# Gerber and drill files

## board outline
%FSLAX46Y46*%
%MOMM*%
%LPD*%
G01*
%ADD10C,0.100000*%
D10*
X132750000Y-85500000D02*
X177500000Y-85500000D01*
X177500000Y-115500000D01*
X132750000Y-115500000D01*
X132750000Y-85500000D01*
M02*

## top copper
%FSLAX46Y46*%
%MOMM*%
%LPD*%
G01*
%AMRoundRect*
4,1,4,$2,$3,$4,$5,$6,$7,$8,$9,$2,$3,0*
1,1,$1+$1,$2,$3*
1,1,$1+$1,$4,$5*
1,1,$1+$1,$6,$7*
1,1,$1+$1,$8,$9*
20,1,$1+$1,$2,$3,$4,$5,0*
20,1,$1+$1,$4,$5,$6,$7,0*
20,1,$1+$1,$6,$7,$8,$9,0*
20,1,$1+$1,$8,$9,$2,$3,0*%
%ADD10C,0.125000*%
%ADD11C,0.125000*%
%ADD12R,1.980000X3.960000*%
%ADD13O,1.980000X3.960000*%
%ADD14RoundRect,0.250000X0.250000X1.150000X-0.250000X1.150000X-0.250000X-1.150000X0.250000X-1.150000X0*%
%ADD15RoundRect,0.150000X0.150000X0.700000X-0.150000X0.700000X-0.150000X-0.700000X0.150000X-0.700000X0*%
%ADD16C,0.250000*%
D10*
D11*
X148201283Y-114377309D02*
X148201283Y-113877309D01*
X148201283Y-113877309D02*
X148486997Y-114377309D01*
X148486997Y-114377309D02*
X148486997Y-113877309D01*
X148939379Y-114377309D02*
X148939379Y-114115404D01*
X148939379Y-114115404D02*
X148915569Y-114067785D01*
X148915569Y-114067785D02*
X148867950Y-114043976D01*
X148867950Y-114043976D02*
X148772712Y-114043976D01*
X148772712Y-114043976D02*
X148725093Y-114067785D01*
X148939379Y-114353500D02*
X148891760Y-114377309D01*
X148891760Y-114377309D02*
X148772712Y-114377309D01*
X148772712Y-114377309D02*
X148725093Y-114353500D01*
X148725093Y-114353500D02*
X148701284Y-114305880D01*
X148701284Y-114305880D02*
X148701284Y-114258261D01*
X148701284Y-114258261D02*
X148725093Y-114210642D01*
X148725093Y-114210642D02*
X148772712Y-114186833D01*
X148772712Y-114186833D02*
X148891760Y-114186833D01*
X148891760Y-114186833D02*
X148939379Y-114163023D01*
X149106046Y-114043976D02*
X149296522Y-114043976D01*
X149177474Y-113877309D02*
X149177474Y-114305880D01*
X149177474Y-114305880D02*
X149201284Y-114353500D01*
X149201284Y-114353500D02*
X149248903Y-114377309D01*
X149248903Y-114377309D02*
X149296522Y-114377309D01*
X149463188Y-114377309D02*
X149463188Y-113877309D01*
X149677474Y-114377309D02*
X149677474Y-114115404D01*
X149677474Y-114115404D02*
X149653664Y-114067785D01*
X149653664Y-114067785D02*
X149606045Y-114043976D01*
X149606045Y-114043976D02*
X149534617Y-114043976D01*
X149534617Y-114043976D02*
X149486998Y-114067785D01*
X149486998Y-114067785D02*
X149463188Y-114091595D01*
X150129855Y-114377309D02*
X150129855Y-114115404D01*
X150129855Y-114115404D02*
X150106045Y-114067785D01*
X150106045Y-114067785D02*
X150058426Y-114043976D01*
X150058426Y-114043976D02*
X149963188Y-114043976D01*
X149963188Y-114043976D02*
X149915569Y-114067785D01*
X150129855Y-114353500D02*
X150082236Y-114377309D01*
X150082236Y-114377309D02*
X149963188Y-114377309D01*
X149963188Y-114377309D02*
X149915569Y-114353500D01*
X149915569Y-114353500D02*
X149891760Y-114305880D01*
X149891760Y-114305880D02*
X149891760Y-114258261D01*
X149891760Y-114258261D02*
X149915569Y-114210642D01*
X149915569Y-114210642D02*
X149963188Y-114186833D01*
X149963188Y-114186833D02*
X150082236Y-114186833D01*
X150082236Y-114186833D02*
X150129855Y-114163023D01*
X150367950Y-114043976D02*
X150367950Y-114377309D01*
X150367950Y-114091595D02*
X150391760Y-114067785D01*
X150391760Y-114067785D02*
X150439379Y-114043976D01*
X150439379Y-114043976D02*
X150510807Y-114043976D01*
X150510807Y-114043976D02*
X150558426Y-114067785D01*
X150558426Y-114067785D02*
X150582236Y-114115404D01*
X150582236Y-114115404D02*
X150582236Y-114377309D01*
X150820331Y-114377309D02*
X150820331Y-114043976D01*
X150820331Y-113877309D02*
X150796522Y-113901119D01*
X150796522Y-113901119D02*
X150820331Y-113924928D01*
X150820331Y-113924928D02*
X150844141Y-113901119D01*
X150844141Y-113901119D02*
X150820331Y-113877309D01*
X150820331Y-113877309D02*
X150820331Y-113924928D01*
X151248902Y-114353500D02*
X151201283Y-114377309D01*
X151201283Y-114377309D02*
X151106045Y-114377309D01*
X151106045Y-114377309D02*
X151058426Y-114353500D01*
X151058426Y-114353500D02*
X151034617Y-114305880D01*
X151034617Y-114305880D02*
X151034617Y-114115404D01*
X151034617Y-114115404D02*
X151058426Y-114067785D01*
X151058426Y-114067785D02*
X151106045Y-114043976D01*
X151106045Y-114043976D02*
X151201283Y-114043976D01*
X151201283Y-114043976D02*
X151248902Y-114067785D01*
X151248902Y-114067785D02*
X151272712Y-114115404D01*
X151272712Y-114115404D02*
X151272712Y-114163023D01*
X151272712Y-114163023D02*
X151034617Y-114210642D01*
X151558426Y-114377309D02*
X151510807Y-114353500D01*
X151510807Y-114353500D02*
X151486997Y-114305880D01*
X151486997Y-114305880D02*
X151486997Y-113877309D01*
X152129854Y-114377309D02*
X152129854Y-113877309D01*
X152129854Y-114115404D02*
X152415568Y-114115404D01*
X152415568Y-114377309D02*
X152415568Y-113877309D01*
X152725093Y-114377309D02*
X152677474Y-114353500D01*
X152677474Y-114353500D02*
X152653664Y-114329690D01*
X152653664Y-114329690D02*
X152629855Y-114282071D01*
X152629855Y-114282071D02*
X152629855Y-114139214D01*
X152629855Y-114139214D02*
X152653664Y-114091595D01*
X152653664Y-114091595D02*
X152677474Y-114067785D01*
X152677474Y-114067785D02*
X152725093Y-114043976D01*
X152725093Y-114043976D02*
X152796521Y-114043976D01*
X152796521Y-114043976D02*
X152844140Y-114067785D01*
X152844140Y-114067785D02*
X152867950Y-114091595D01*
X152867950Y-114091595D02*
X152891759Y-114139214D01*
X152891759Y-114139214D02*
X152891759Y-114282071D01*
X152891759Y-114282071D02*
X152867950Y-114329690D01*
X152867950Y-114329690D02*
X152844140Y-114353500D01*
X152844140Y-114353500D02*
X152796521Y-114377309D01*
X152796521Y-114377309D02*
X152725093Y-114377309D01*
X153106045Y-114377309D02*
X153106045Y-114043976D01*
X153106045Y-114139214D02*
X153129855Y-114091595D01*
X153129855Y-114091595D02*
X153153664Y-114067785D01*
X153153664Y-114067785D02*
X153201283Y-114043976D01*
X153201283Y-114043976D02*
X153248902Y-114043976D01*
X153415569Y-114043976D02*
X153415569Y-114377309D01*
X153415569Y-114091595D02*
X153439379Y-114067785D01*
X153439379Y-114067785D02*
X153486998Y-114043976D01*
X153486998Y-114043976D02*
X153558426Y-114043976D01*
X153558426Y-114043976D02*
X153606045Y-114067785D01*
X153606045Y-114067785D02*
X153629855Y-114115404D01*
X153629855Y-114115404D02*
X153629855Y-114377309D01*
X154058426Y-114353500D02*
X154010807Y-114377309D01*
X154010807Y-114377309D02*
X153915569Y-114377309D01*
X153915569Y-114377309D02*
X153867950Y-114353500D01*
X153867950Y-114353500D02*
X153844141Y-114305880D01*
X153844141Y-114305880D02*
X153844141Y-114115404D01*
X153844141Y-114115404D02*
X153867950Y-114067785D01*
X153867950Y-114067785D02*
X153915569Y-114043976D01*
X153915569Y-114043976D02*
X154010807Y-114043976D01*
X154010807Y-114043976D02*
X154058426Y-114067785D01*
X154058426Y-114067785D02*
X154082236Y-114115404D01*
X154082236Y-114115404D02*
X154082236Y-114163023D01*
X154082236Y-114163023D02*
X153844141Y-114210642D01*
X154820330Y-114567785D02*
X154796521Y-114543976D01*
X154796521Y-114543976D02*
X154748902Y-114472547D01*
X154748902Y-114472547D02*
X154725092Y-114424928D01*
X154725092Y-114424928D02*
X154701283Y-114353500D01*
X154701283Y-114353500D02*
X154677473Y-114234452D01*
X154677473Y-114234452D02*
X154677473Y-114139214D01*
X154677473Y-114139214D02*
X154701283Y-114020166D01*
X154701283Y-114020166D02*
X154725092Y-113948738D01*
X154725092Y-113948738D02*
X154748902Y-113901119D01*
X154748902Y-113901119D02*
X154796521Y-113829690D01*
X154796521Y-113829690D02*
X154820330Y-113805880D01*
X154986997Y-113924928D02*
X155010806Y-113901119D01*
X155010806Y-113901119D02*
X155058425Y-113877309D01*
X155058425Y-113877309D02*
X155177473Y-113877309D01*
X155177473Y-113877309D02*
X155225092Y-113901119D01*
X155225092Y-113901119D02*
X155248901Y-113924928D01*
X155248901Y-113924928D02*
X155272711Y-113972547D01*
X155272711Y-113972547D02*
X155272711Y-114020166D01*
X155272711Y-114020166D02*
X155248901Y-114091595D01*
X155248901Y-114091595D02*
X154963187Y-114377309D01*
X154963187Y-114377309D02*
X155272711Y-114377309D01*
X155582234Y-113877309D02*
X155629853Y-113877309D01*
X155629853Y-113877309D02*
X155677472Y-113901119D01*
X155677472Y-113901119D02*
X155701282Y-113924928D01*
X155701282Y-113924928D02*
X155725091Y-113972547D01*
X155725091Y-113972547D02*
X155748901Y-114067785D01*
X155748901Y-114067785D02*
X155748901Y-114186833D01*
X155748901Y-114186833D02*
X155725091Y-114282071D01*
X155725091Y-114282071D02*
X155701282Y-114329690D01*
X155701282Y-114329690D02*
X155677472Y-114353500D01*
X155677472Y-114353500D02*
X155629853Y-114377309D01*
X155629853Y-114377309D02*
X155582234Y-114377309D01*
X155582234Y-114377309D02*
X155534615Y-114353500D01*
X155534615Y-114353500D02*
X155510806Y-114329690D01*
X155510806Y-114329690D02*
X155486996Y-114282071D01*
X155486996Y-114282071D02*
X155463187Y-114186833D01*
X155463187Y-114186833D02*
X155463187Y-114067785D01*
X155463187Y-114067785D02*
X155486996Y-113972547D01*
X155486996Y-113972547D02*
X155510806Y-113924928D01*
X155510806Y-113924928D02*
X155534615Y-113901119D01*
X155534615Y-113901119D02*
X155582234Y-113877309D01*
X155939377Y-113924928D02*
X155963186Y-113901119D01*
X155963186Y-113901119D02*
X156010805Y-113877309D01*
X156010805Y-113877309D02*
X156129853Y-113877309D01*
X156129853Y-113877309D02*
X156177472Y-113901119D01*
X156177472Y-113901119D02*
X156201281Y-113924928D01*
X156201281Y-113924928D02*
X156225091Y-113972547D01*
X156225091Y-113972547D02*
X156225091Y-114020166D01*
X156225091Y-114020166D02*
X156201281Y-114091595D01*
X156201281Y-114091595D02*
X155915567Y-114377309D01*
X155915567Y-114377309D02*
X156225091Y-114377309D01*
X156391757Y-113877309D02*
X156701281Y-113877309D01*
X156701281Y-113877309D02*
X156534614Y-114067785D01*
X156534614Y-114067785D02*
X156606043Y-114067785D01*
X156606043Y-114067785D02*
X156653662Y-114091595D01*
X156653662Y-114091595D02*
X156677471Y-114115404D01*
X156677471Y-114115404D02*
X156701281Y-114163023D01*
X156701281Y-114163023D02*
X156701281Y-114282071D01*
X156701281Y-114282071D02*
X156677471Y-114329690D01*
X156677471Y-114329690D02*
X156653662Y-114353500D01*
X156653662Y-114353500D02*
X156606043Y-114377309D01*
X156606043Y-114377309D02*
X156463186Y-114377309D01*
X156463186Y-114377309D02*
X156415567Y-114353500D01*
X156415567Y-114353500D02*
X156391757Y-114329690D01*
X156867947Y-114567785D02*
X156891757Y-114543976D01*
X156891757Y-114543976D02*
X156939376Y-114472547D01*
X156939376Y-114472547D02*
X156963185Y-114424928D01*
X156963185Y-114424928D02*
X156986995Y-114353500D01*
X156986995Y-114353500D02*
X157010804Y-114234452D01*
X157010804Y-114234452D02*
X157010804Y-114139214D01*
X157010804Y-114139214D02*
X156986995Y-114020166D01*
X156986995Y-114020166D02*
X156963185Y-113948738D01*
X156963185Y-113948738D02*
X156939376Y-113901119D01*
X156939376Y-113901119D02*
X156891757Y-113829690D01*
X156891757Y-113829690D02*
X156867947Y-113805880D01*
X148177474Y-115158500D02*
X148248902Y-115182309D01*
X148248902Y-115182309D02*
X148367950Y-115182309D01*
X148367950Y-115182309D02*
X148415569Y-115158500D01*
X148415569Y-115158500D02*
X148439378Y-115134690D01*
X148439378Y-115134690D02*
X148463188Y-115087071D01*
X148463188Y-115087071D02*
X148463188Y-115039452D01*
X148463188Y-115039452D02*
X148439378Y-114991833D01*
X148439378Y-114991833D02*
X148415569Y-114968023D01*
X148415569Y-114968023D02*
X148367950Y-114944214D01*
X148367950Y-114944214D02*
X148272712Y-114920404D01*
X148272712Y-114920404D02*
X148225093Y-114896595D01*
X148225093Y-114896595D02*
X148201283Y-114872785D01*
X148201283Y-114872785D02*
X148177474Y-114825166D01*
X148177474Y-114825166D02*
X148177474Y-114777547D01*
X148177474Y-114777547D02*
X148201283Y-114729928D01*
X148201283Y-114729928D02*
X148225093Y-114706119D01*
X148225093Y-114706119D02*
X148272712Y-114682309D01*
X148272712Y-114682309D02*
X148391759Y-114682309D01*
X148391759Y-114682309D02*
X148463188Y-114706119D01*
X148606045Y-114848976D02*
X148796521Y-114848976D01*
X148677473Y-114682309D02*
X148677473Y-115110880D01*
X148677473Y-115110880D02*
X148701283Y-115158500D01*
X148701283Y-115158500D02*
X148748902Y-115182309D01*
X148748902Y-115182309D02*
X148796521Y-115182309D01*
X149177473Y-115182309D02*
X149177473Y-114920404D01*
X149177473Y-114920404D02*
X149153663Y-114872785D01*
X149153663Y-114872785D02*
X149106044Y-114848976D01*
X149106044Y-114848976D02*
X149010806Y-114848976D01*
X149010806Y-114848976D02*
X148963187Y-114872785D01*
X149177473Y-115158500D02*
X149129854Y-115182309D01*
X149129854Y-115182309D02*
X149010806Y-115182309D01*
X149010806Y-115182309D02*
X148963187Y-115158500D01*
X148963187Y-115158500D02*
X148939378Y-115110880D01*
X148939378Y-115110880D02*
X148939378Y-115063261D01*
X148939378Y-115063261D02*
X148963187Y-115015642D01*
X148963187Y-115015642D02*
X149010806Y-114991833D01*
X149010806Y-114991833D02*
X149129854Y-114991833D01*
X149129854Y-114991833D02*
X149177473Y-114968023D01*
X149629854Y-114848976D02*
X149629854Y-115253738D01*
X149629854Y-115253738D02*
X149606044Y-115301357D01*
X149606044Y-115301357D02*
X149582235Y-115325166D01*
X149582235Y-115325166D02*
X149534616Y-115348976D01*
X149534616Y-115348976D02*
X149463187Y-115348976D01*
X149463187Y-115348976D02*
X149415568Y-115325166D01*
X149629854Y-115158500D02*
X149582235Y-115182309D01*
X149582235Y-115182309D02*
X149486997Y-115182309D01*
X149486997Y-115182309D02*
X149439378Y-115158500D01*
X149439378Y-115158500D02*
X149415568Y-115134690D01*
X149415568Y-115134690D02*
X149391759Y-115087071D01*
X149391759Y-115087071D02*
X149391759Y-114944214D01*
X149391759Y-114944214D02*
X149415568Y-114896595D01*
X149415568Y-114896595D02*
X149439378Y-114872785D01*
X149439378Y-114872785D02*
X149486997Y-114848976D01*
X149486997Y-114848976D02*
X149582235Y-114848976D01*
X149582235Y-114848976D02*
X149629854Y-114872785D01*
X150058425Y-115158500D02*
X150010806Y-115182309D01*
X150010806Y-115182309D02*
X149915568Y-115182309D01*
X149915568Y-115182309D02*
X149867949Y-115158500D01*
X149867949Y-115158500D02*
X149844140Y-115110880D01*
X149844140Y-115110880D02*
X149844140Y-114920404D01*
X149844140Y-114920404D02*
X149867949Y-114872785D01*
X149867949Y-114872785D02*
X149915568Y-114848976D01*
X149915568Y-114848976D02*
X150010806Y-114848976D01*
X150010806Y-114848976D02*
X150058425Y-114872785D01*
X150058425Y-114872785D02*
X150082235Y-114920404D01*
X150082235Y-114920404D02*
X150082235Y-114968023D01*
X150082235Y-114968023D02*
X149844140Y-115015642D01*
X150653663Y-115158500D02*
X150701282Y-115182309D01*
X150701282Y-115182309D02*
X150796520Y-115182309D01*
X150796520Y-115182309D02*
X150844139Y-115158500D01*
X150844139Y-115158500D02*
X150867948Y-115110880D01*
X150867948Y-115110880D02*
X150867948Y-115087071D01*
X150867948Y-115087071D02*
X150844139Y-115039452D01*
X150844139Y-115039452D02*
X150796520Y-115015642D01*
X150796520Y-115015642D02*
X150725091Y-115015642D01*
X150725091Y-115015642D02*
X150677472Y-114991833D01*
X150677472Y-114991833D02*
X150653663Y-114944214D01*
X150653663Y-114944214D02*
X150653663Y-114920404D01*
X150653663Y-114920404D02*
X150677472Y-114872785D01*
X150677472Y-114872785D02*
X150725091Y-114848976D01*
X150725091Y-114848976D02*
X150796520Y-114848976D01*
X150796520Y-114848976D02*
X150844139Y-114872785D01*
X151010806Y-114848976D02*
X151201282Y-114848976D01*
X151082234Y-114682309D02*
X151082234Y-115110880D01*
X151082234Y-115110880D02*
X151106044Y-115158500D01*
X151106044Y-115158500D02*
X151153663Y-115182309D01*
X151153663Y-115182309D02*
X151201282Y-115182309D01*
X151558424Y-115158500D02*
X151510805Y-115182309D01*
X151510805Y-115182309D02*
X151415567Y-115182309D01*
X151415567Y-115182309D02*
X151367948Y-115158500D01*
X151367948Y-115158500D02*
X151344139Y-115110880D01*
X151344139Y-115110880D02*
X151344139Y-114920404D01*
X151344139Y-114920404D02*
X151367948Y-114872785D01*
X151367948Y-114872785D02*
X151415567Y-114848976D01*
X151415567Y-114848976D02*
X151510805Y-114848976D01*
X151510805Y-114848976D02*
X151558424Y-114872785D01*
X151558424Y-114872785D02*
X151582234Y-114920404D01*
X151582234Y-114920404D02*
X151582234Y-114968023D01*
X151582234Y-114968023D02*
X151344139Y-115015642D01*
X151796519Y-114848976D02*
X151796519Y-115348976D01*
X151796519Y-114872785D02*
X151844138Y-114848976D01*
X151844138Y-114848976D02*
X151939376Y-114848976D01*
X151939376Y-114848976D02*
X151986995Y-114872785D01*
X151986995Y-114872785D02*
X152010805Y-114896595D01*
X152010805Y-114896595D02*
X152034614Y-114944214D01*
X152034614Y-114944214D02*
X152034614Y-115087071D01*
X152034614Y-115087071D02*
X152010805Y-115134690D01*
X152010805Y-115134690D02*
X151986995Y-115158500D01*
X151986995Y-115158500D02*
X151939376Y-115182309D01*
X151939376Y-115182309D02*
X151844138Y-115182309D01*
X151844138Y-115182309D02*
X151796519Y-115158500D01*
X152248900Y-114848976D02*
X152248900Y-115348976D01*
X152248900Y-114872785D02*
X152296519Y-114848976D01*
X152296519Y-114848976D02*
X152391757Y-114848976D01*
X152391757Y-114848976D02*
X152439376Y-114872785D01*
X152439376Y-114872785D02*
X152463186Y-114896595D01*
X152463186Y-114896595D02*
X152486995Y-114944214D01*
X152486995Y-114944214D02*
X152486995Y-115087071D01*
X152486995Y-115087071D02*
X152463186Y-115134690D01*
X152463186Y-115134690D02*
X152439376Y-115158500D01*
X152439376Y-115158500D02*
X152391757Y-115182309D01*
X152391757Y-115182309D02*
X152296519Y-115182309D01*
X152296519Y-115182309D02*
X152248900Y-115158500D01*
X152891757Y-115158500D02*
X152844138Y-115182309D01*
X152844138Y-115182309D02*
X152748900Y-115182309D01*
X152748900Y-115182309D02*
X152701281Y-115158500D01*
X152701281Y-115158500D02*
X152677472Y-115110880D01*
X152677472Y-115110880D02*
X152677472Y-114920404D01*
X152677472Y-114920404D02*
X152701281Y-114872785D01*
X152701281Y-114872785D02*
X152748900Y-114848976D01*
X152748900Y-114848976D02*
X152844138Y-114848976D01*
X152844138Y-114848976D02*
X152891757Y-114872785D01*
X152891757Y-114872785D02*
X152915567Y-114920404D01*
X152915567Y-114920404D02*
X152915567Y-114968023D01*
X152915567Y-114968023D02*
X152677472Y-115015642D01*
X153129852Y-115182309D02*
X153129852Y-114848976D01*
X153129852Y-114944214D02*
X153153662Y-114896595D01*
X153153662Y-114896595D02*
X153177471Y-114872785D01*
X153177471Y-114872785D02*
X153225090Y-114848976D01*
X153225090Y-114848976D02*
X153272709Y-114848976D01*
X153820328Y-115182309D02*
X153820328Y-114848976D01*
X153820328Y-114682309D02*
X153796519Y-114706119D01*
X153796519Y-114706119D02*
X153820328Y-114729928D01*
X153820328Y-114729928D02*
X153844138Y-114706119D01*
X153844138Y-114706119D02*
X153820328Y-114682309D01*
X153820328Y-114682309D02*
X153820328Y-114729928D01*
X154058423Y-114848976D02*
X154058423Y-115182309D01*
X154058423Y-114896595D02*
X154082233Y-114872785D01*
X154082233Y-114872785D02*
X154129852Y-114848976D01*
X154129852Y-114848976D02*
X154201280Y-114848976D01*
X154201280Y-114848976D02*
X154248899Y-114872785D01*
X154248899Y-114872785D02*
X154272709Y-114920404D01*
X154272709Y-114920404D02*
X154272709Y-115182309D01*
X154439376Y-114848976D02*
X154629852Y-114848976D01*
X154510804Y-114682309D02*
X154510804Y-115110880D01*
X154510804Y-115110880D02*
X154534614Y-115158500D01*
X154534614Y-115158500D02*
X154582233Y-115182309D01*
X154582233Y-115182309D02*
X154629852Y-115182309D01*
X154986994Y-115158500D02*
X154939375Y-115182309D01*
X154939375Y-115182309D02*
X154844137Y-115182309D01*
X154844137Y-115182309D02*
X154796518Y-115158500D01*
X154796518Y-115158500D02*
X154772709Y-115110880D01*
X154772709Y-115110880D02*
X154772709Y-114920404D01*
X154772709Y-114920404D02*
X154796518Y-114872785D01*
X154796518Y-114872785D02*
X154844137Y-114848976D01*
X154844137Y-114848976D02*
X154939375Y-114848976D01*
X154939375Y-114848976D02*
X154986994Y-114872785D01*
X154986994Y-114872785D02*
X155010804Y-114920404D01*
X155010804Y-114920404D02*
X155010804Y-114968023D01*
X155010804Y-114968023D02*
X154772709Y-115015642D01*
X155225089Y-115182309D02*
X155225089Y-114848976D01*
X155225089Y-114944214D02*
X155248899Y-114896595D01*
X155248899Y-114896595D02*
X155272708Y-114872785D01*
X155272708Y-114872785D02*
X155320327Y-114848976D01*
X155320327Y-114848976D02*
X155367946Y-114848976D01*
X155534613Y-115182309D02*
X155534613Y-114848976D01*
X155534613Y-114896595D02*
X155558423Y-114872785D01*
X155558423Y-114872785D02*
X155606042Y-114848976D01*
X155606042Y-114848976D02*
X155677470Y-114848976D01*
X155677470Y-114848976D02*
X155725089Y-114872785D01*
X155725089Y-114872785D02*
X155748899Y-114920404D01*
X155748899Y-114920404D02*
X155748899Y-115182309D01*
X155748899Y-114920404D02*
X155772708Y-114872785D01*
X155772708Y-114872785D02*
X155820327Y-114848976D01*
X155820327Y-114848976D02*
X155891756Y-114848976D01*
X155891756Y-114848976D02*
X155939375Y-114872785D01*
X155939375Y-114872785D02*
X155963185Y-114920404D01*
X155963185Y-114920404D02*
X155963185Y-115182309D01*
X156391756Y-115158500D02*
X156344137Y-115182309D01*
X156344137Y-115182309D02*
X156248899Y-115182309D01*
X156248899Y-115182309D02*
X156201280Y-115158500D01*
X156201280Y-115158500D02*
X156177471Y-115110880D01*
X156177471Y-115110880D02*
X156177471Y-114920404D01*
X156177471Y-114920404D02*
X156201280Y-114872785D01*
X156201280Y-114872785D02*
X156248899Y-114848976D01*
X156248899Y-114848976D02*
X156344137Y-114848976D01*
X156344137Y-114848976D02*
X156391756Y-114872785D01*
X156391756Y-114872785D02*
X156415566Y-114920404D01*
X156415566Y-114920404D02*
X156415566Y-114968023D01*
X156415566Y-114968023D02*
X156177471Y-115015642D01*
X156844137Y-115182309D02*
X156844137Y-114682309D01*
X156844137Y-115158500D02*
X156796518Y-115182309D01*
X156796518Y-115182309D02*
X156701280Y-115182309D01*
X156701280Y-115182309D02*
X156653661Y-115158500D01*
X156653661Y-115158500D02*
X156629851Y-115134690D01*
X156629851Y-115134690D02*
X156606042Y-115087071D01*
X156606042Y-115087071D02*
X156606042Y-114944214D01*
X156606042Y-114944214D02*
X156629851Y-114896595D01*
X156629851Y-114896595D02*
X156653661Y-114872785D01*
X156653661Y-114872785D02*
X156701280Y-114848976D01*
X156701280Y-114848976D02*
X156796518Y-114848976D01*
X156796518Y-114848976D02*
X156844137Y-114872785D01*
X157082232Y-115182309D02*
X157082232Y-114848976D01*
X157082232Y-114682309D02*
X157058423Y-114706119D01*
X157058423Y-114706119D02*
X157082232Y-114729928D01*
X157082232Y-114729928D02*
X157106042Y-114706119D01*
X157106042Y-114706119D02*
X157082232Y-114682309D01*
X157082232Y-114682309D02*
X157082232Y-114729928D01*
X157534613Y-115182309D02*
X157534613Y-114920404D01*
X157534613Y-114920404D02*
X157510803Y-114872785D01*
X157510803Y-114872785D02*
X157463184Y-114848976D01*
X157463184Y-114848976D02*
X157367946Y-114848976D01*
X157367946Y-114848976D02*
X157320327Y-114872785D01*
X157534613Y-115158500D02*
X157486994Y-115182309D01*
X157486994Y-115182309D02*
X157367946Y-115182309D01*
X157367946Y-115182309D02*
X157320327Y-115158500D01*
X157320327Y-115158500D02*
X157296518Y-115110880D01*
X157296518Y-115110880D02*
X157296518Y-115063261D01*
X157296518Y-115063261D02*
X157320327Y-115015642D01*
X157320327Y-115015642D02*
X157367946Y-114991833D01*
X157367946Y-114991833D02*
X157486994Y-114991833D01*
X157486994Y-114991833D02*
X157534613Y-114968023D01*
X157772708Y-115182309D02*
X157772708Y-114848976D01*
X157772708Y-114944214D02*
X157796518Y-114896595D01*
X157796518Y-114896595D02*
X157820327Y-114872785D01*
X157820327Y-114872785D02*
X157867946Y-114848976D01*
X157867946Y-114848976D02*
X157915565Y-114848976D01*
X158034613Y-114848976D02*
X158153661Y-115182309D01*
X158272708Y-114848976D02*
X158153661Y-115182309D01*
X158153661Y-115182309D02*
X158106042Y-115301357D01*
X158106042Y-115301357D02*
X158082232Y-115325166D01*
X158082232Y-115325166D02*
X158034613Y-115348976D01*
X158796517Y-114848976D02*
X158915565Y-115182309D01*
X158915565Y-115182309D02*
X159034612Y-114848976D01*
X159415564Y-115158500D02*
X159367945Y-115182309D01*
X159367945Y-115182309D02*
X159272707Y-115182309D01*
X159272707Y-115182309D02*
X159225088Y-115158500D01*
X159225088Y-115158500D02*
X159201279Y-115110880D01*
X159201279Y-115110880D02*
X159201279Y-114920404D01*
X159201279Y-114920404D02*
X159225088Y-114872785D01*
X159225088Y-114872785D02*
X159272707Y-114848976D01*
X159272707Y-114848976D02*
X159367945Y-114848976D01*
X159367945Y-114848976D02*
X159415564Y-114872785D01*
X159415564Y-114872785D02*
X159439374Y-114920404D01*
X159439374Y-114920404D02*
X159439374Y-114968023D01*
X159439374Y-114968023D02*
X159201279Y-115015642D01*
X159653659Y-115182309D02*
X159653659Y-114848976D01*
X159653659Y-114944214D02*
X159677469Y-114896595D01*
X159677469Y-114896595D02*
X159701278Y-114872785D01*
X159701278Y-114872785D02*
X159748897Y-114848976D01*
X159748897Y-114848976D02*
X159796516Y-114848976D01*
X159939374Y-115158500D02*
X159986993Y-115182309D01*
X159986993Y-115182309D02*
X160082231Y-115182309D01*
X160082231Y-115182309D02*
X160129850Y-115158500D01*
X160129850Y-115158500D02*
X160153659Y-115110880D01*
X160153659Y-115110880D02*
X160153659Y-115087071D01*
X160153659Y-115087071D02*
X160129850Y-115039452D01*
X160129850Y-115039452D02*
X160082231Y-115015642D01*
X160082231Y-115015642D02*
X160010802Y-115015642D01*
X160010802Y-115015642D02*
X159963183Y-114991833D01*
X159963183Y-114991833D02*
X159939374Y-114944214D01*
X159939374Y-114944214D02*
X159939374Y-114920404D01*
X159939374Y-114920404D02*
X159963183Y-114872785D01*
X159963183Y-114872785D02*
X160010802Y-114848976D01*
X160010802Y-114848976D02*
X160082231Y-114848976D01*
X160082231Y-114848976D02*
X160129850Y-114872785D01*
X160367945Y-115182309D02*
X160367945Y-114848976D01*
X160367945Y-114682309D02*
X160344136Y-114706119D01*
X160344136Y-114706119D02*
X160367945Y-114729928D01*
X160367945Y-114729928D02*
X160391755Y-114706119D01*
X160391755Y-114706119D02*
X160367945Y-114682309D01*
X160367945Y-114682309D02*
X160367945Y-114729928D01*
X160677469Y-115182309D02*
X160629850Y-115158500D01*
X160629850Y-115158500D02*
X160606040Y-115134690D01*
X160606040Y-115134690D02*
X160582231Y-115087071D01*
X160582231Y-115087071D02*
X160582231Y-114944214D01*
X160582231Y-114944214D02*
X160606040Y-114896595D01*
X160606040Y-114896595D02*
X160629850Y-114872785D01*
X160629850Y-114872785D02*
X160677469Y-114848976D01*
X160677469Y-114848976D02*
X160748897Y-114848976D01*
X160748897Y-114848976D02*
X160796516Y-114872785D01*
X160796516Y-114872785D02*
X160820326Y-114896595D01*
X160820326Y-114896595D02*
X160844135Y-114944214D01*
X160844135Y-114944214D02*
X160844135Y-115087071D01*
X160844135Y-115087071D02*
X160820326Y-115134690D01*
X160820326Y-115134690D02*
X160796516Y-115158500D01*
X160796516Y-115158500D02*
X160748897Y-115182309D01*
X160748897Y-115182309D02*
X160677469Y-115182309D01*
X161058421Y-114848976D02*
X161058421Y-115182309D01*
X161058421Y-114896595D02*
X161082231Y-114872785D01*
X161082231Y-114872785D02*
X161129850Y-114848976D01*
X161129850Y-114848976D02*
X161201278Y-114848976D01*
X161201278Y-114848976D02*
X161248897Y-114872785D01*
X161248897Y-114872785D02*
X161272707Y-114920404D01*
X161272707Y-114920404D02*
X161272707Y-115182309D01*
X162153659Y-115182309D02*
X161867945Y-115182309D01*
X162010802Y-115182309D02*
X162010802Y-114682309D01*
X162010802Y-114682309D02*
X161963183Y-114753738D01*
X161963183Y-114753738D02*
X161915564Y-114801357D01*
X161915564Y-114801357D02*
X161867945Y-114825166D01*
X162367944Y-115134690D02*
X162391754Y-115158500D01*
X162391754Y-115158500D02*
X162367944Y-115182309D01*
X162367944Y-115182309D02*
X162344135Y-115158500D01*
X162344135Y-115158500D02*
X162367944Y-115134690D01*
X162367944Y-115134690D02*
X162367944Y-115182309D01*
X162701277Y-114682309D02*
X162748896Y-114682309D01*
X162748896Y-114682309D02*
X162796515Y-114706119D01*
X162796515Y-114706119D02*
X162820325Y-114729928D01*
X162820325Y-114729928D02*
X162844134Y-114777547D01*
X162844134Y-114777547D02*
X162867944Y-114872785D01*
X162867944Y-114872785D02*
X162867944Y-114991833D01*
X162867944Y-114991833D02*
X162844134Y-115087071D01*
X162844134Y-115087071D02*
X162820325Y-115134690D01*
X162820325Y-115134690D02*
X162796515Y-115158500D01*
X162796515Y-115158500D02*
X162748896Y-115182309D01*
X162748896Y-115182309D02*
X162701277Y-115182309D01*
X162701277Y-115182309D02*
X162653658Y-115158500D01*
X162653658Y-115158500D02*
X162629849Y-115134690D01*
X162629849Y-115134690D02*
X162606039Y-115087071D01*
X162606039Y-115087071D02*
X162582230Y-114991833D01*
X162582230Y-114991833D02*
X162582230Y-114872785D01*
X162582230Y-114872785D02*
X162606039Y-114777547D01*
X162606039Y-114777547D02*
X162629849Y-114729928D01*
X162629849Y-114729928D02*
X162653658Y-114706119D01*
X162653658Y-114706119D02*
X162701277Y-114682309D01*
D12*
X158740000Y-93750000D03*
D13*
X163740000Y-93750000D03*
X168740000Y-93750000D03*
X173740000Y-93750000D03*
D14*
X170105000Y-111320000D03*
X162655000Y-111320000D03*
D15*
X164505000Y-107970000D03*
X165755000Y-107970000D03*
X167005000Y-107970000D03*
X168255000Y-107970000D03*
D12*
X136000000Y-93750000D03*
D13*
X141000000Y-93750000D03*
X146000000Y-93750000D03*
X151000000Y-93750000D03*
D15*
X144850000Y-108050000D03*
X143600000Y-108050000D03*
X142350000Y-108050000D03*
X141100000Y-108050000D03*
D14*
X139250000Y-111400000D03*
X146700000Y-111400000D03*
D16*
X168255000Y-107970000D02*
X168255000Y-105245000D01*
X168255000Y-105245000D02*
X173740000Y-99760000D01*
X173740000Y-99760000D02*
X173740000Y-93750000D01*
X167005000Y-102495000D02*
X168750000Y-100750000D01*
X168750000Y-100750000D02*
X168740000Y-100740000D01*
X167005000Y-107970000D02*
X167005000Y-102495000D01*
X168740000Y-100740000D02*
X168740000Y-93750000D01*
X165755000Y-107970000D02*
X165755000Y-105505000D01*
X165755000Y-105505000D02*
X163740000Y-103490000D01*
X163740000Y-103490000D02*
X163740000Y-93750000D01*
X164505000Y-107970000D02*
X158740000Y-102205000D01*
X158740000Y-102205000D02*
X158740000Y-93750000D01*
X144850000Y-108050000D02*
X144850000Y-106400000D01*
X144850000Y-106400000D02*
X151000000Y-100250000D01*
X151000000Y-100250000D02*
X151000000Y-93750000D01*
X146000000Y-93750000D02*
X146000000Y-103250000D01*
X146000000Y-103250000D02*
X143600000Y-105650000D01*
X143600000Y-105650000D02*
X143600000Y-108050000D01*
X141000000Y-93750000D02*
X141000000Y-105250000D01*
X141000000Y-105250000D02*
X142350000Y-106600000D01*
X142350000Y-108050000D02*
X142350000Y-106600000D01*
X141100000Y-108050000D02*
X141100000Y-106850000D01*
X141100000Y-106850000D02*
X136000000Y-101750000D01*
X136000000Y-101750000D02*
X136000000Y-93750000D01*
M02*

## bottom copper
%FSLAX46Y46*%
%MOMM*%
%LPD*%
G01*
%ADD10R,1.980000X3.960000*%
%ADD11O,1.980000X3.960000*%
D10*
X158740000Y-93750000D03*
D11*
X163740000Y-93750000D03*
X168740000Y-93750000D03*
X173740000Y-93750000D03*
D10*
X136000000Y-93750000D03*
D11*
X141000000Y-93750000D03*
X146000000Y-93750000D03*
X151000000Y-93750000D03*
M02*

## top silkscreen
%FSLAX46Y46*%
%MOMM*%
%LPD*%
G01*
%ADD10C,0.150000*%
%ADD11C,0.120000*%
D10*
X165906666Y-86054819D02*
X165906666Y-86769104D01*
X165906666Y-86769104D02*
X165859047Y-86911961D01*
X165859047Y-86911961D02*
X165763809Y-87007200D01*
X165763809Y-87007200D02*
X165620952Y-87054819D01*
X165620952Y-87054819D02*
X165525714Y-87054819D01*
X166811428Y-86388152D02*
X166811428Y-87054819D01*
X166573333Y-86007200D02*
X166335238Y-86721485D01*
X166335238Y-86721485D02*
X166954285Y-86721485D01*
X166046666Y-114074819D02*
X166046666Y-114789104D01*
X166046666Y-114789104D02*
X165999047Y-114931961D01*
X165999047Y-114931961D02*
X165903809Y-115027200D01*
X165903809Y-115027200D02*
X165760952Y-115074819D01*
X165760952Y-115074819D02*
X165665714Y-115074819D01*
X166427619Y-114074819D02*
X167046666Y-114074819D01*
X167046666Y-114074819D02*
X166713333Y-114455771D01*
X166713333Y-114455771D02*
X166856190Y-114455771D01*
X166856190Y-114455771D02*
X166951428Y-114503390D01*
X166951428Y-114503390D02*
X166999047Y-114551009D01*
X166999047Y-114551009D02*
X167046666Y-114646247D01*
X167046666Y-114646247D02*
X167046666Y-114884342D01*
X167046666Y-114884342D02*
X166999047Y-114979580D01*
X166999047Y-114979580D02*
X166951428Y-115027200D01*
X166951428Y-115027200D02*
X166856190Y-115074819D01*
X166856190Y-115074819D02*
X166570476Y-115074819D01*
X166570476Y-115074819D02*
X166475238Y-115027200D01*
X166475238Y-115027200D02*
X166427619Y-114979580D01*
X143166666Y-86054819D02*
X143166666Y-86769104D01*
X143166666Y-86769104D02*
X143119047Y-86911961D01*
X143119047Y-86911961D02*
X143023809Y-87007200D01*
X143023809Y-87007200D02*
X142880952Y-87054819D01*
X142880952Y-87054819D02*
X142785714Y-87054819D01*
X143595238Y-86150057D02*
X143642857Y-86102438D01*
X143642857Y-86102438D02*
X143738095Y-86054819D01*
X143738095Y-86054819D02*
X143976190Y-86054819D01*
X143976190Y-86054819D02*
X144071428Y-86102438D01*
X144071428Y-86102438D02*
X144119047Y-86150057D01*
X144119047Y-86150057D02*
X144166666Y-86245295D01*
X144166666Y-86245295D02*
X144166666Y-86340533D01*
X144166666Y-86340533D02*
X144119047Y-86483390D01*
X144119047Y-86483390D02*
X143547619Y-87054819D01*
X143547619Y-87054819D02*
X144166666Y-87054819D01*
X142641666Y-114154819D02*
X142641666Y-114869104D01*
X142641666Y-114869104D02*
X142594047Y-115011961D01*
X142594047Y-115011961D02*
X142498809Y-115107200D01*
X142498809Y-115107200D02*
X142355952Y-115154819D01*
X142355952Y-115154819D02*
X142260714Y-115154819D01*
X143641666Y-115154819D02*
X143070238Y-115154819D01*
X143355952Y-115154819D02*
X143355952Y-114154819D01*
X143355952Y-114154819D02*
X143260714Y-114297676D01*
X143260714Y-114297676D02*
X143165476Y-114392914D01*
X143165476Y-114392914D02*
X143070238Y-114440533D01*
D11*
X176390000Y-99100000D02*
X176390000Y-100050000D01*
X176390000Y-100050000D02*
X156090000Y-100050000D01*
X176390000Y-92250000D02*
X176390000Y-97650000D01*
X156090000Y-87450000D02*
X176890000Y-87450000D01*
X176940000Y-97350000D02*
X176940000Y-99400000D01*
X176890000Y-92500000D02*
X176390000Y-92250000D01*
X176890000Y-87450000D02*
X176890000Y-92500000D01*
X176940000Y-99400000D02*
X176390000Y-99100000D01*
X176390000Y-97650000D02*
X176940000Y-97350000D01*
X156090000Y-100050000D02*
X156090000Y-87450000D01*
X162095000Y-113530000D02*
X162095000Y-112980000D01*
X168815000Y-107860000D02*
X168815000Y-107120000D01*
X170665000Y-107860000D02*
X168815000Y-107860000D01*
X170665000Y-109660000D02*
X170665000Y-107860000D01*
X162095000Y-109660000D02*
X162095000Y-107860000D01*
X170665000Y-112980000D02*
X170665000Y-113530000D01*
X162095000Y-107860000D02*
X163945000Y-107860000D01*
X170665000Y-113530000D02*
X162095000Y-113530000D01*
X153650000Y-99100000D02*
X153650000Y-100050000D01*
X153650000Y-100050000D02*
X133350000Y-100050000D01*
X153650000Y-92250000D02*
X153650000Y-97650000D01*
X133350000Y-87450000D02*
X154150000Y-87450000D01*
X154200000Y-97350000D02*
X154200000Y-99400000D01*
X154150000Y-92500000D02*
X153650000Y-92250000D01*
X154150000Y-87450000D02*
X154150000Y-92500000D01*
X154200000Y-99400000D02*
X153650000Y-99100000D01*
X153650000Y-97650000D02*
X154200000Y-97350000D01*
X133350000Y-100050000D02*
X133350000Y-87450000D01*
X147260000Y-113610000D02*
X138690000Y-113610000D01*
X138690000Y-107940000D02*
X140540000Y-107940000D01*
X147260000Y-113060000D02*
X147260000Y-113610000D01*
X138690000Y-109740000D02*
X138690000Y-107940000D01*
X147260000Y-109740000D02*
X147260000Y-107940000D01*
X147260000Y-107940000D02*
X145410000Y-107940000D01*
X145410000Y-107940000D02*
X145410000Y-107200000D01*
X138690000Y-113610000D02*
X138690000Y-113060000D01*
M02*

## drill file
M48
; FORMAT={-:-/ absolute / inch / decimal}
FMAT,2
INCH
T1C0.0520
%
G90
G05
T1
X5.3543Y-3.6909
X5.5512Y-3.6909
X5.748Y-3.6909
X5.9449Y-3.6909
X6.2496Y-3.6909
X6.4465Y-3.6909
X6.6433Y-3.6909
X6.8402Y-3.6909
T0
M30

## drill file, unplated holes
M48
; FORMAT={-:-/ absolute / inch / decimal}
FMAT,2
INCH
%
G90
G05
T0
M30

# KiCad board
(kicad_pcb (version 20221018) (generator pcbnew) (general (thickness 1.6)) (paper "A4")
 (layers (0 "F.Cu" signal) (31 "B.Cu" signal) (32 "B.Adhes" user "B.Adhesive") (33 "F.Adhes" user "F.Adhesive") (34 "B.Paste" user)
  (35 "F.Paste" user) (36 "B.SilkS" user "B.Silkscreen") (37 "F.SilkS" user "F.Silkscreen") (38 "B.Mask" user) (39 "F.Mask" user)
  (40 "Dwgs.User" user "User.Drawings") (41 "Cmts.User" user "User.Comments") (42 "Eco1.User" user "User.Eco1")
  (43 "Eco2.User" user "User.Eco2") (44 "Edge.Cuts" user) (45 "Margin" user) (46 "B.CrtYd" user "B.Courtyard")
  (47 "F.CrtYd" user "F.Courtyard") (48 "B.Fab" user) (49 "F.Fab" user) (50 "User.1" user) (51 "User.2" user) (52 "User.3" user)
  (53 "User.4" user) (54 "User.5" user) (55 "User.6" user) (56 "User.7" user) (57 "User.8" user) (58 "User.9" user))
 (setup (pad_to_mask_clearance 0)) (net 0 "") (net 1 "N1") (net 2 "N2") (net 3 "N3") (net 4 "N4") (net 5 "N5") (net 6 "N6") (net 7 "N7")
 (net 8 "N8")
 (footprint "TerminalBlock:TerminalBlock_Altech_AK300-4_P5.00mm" (layer "F.Cu") (at 136 93.75)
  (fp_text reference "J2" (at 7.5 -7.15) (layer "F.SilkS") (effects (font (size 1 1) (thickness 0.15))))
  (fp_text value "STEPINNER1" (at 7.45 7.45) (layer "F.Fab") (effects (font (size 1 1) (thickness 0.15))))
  (fp_line (start -2.65 -6.3) (end 18.15 -6.3) (stroke (width 0.12) (type solid)) (layer "F.SilkS"))
  (fp_line (start -2.65 6.3) (end -2.65 -6.3) (stroke (width 0.12) (type solid)) (layer "F.SilkS"))
  (fp_line (start 17.65 -1.5) (end 17.65 3.9) (stroke (width 0.12) (type solid)) (layer "F.SilkS"))
  (fp_line (start 17.65 3.9) (end 18.2 3.6) (stroke (width 0.12) (type solid)) (layer "F.SilkS"))
  (fp_line (start 17.65 5.35) (end 17.65 6.3) (stroke (width 0.12) (type solid)) (layer "F.SilkS"))
  (fp_line (start 17.65 6.3) (end -2.65 6.3) (stroke (width 0.12) (type solid)) (layer "F.SilkS"))
  (fp_line (start 18.15 -6.3) (end 18.15 -1.25) (stroke (width 0.12) (type solid)) (layer "F.SilkS"))
  (fp_line (start 18.15 -1.25) (end 17.65 -1.5) (stroke (width 0.12) (type solid)) (layer "F.SilkS"))
  (fp_line (start 18.2 3.6) (end 18.2 5.65) (stroke (width 0.12) (type solid)) (layer "F.SilkS"))
  (fp_line (start 18.2 5.65) (end 17.65 5.35) (stroke (width 0.12) (type solid)) (layer "F.SilkS"))
  (pad "1" thru_hole rect (at 0 0) (size 1.98 3.96) (drill 1.32) (layers "*.Cu" "*.Mask") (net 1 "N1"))
  (pad "2" thru_hole oval (at 5 0) (size 1.98 3.96) (drill 1.32) (layers "*.Cu" "*.Mask") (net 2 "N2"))
  (pad "3" thru_hole oval (at 10 0) (size 1.98 3.96) (drill 1.32) (layers "*.Cu" "*.Mask") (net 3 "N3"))
  (pad "4" thru_hole oval (at 15 0) (size 1.98 3.96) (drill 1.32) (layers "*.Cu" "*.Mask") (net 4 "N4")))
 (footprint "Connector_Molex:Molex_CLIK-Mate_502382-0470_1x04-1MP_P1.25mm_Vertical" (layer "F.Cu") (at 142.975 110 180)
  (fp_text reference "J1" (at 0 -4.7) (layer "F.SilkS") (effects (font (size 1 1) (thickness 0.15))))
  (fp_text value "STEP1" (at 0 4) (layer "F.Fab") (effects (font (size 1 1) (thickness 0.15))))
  (fp_line (start -4.285 -3.61) (end 4.285 -3.61) (stroke (width 0.12) (type solid)) (layer "F.SilkS"))
  (fp_line (start -4.285 -3.06) (end -4.285 -3.61) (stroke (width 0.12) (type solid)) (layer "F.SilkS"))
  (fp_line (start -4.285 0.26) (end -4.285 2.06) (stroke (width 0.12) (type solid)) (layer "F.SilkS"))
  (fp_line (start -4.285 2.06) (end -2.435 2.06) (stroke (width 0.12) (type solid)) (layer "F.SilkS"))
  (fp_line (start -2.435 2.06) (end -2.435 2.8) (stroke (width 0.12) (type solid)) (layer "F.SilkS"))
  (fp_line (start 4.285 -3.61) (end 4.285 -3.06) (stroke (width 0.12) (type solid)) (layer "F.SilkS"))
  (fp_line (start 4.285 0.26) (end 4.285 2.06) (stroke (width 0.12) (type solid)) (layer "F.SilkS"))
  (fp_line (start 4.285 2.06) (end 2.435 2.06) (stroke (width 0.12) (type solid)) (layer "F.SilkS"))
  (pad "1" smd roundrect (at -1.875 1.95 180) (size 0.6 1.7) (layers "F.Cu" "F.Paste" "F.Mask") (roundrect_rratio 0.25) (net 4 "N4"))
  (pad "2" smd roundrect (at -0.625 1.95 180) (size 0.6 1.7) (layers "F.Cu" "F.Paste" "F.Mask") (roundrect_rratio 0.25) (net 3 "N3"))
  (pad "3" smd roundrect (at 0.625 1.95 180) (size 0.6 1.7) (layers "F.Cu" "F.Paste" "F.Mask") (roundrect_rratio 0.25) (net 2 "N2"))
  (pad "4" smd roundrect (at 1.875 1.95 180) (size 0.6 1.7) (layers "F.Cu" "F.Paste" "F.Mask") (roundrect_rratio 0.25) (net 1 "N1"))
  (pad "MP" smd roundrect (at -3.725 -1.4 180) (size 1 2.8) (layers "F.Cu" "F.Paste" "F.Mask") (roundrect_rratio 0.25))
  (pad "MP" smd roundrect (at 3.725 -1.4 180) (size 1 2.8) (layers "F.Cu" "F.Paste" "F.Mask") (roundrect_rratio 0.25)))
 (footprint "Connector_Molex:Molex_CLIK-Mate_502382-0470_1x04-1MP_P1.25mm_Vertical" (layer "F.Cu") (at 166.38 109.92 180)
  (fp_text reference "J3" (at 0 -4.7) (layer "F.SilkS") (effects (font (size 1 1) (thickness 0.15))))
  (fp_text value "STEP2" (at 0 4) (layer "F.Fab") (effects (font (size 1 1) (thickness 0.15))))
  (fp_line (start -4.285 -3.61) (end 4.285 -3.61) (stroke (width 0.12) (type solid)) (layer "F.SilkS"))
  (fp_line (start -4.285 -3.06) (end -4.285 -3.61) (stroke (width 0.12) (type solid)) (layer "F.SilkS"))
  (fp_line (start -4.285 0.26) (end -4.285 2.06) (stroke (width 0.12) (type solid)) (layer "F.SilkS"))
  (fp_line (start -4.285 2.06) (end -2.435 2.06) (stroke (width 0.12) (type solid)) (layer "F.SilkS"))
  (fp_line (start -2.435 2.06) (end -2.435 2.8) (stroke (width 0.12) (type solid)) (layer "F.SilkS"))
  (fp_line (start 4.285 -3.61) (end 4.285 -3.06) (stroke (width 0.12) (type solid)) (layer "F.SilkS"))
  (fp_line (start 4.285 0.26) (end 4.285 2.06) (stroke (width 0.12) (type solid)) (layer "F.SilkS"))
  (fp_line (start 4.285 2.06) (end 2.435 2.06) (stroke (width 0.12) (type solid)) (layer "F.SilkS"))
  (pad "1" smd roundrect (at -1.875 1.95 180) (size 0.6 1.7) (layers "F.Cu" "F.Paste" "F.Mask") (roundrect_rratio 0.25) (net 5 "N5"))
  (pad "2" smd roundrect (at -0.625 1.95 180) (size 0.6 1.7) (layers "F.Cu" "F.Paste" "F.Mask") (roundrect_rratio 0.25) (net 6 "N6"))
  (pad "3" smd roundrect (at 0.625 1.95 180) (size 0.6 1.7) (layers "F.Cu" "F.Paste" "F.Mask") (roundrect_rratio 0.25) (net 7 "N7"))
  (pad "4" smd roundrect (at 1.875 1.95 180) (size 0.6 1.7) (layers "F.Cu" "F.Paste" "F.Mask") (roundrect_rratio 0.25) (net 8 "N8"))
  (pad "MP" smd roundrect (at -3.725 -1.4 180) (size 1 2.8) (layers "F.Cu" "F.Paste" "F.Mask") (roundrect_rratio 0.25))
  (pad "MP" smd roundrect (at 3.725 -1.4 180) (size 1 2.8) (layers "F.Cu" "F.Paste" "F.Mask") (roundrect_rratio 0.25)))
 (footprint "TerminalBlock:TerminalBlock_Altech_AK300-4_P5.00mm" (layer "F.Cu") (at 158.74 93.75)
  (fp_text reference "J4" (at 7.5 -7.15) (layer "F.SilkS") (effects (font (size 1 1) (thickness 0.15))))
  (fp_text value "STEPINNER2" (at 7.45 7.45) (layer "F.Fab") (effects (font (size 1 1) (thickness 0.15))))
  (fp_line (start -2.65 -6.3) (end 18.15 -6.3) (stroke (width 0.12) (type solid)) (layer "F.SilkS"))
  (fp_line (start -2.65 6.3) (end -2.65 -6.3) (stroke (width 0.12) (type solid)) (layer "F.SilkS"))
  (fp_line (start 17.65 -1.5) (end 17.65 3.9) (stroke (width 0.12) (type solid)) (layer "F.SilkS"))
  (fp_line (start 17.65 3.9) (end 18.2 3.6) (stroke (width 0.12) (type solid)) (layer "F.SilkS"))
  (fp_line (start 17.65 5.35) (end 17.65 6.3) (stroke (width 0.12) (type solid)) (layer "F.SilkS"))
  (fp_line (start 17.65 6.3) (end -2.65 6.3) (stroke (width 0.12) (type solid)) (layer "F.SilkS"))
  (fp_line (start 18.15 -6.3) (end 18.15 -1.25) (stroke (width 0.12) (type solid)) (layer "F.SilkS"))
  (fp_line (start 18.15 -1.25) (end 17.65 -1.5) (stroke (width 0.12) (type solid)) (layer "F.SilkS"))
  (fp_line (start 18.2 3.6) (end 18.2 5.65) (stroke (width 0.12) (type solid)) (layer "F.SilkS"))
  (fp_line (start 18.2 5.65) (end 17.65 5.35) (stroke (width 0.12) (type solid)) (layer "F.SilkS"))
  (pad "1" thru_hole rect (at 0 0) (size 1.98 3.96) (drill 1.32) (layers "*.Cu" "*.Mask") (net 8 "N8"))
  (pad "2" thru_hole oval (at 5 0) (size 1.98 3.96) (drill 1.32) (layers "*.Cu" "*.Mask") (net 7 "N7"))
  (pad "3" thru_hole oval (at 10 0) (size 1.98 3.96) (drill 1.32) (layers "*.Cu" "*.Mask") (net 6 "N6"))
  (pad "4" thru_hole oval (at 15 0) (size 1.98 3.96) (drill 1.32) (layers "*.Cu" "*.Mask") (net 5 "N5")))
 (gr_rect (start 132.75 85.5) (end 177.5 115.5) (stroke (width 0.1) (type default)) (fill none) (layer "Edge.Cuts"))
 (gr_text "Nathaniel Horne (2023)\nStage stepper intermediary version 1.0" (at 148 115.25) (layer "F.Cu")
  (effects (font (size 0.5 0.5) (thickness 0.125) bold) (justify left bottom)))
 (segment (start 144.85 108.05) (end 144.85 106.4) (width 0.25) (layer "F.Cu") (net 4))
 (segment (start 151 100.25) (end 151 93.75) (width 0.25) (layer "F.Cu") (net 4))
 (segment (start 144.85 106.4) (end 151 100.25) (width 0.25) (layer "F.Cu") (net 4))
 (segment (start 143.6 105.65) (end 143.6 108.05) (width 0.25) (layer "F.Cu") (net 3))
 (segment (start 146 93.75) (end 146 103.25) (width 0.25) (layer "F.Cu") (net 3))
 (segment (start 146 103.25) (end 143.6 105.65) (width 0.25) (layer "F.Cu") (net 3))
 (segment (start 142.35 108.05) (end 142.35 106.6) (width 0.25) (layer "F.Cu") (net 2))
 (segment (start 141 105.25) (end 142.35 106.6) (width 0.25) (layer "F.Cu") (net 2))
 (segment (start 141 93.75) (end 141 105.25) (width 0.25) (layer "F.Cu") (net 2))
 (segment (start 141.1 106.85) (end 136 101.75) (width 0.25) (layer "F.Cu") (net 1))
 (segment (start 141.1 108.05) (end 141.1 106.85) (width 0.25) (layer "F.Cu") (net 1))
 (segment (start 136 101.75) (end 136 93.75) (width 0.25) (layer "F.Cu") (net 1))
 (segment (start 173.74 99.76) (end 173.74 93.75) (width 0.25) (layer "F.Cu") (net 5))
 (segment (start 168.255 107.97) (end 168.255 105.245) (width 0.25) (layer "F.Cu") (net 5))
 (segment (start 168.255 105.245) (end 173.74 99.76) (width 0.25) (layer "F.Cu") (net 5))
 (segment (start 168.74 100.74) (end 168.74 93.75) (width 0.25) (layer "F.Cu") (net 6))
 (segment (start 167.005 107.97) (end 167.005 102.495) (width 0.25) (layer "F.Cu") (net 6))
 (segment (start 167.005 102.495) (end 168.75 100.75) (width 0.25) (layer "F.Cu") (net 6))
 (segment (start 168.75 100.75) (end 168.74 100.74) (width 0.25) (layer "F.Cu") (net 6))
 (segment (start 165.755 107.97) (end 165.755 105.505) (width 0.25) (layer "F.Cu") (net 7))
 (segment (start 163.74 103.49) (end 163.74 93.75) (width 0.25) (layer "F.Cu") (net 7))
 (segment (start 165.755 105.505) (end 163.74 103.49) (width 0.25) (layer "F.Cu") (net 7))
 (segment (start 158.74 102.205) (end 158.74 93.75) (width 0.25) (layer "F.Cu") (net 8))
 (segment (start 164.505 107.97) (end 158.74 102.205) (width 0.25) (layer "F.Cu") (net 8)))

